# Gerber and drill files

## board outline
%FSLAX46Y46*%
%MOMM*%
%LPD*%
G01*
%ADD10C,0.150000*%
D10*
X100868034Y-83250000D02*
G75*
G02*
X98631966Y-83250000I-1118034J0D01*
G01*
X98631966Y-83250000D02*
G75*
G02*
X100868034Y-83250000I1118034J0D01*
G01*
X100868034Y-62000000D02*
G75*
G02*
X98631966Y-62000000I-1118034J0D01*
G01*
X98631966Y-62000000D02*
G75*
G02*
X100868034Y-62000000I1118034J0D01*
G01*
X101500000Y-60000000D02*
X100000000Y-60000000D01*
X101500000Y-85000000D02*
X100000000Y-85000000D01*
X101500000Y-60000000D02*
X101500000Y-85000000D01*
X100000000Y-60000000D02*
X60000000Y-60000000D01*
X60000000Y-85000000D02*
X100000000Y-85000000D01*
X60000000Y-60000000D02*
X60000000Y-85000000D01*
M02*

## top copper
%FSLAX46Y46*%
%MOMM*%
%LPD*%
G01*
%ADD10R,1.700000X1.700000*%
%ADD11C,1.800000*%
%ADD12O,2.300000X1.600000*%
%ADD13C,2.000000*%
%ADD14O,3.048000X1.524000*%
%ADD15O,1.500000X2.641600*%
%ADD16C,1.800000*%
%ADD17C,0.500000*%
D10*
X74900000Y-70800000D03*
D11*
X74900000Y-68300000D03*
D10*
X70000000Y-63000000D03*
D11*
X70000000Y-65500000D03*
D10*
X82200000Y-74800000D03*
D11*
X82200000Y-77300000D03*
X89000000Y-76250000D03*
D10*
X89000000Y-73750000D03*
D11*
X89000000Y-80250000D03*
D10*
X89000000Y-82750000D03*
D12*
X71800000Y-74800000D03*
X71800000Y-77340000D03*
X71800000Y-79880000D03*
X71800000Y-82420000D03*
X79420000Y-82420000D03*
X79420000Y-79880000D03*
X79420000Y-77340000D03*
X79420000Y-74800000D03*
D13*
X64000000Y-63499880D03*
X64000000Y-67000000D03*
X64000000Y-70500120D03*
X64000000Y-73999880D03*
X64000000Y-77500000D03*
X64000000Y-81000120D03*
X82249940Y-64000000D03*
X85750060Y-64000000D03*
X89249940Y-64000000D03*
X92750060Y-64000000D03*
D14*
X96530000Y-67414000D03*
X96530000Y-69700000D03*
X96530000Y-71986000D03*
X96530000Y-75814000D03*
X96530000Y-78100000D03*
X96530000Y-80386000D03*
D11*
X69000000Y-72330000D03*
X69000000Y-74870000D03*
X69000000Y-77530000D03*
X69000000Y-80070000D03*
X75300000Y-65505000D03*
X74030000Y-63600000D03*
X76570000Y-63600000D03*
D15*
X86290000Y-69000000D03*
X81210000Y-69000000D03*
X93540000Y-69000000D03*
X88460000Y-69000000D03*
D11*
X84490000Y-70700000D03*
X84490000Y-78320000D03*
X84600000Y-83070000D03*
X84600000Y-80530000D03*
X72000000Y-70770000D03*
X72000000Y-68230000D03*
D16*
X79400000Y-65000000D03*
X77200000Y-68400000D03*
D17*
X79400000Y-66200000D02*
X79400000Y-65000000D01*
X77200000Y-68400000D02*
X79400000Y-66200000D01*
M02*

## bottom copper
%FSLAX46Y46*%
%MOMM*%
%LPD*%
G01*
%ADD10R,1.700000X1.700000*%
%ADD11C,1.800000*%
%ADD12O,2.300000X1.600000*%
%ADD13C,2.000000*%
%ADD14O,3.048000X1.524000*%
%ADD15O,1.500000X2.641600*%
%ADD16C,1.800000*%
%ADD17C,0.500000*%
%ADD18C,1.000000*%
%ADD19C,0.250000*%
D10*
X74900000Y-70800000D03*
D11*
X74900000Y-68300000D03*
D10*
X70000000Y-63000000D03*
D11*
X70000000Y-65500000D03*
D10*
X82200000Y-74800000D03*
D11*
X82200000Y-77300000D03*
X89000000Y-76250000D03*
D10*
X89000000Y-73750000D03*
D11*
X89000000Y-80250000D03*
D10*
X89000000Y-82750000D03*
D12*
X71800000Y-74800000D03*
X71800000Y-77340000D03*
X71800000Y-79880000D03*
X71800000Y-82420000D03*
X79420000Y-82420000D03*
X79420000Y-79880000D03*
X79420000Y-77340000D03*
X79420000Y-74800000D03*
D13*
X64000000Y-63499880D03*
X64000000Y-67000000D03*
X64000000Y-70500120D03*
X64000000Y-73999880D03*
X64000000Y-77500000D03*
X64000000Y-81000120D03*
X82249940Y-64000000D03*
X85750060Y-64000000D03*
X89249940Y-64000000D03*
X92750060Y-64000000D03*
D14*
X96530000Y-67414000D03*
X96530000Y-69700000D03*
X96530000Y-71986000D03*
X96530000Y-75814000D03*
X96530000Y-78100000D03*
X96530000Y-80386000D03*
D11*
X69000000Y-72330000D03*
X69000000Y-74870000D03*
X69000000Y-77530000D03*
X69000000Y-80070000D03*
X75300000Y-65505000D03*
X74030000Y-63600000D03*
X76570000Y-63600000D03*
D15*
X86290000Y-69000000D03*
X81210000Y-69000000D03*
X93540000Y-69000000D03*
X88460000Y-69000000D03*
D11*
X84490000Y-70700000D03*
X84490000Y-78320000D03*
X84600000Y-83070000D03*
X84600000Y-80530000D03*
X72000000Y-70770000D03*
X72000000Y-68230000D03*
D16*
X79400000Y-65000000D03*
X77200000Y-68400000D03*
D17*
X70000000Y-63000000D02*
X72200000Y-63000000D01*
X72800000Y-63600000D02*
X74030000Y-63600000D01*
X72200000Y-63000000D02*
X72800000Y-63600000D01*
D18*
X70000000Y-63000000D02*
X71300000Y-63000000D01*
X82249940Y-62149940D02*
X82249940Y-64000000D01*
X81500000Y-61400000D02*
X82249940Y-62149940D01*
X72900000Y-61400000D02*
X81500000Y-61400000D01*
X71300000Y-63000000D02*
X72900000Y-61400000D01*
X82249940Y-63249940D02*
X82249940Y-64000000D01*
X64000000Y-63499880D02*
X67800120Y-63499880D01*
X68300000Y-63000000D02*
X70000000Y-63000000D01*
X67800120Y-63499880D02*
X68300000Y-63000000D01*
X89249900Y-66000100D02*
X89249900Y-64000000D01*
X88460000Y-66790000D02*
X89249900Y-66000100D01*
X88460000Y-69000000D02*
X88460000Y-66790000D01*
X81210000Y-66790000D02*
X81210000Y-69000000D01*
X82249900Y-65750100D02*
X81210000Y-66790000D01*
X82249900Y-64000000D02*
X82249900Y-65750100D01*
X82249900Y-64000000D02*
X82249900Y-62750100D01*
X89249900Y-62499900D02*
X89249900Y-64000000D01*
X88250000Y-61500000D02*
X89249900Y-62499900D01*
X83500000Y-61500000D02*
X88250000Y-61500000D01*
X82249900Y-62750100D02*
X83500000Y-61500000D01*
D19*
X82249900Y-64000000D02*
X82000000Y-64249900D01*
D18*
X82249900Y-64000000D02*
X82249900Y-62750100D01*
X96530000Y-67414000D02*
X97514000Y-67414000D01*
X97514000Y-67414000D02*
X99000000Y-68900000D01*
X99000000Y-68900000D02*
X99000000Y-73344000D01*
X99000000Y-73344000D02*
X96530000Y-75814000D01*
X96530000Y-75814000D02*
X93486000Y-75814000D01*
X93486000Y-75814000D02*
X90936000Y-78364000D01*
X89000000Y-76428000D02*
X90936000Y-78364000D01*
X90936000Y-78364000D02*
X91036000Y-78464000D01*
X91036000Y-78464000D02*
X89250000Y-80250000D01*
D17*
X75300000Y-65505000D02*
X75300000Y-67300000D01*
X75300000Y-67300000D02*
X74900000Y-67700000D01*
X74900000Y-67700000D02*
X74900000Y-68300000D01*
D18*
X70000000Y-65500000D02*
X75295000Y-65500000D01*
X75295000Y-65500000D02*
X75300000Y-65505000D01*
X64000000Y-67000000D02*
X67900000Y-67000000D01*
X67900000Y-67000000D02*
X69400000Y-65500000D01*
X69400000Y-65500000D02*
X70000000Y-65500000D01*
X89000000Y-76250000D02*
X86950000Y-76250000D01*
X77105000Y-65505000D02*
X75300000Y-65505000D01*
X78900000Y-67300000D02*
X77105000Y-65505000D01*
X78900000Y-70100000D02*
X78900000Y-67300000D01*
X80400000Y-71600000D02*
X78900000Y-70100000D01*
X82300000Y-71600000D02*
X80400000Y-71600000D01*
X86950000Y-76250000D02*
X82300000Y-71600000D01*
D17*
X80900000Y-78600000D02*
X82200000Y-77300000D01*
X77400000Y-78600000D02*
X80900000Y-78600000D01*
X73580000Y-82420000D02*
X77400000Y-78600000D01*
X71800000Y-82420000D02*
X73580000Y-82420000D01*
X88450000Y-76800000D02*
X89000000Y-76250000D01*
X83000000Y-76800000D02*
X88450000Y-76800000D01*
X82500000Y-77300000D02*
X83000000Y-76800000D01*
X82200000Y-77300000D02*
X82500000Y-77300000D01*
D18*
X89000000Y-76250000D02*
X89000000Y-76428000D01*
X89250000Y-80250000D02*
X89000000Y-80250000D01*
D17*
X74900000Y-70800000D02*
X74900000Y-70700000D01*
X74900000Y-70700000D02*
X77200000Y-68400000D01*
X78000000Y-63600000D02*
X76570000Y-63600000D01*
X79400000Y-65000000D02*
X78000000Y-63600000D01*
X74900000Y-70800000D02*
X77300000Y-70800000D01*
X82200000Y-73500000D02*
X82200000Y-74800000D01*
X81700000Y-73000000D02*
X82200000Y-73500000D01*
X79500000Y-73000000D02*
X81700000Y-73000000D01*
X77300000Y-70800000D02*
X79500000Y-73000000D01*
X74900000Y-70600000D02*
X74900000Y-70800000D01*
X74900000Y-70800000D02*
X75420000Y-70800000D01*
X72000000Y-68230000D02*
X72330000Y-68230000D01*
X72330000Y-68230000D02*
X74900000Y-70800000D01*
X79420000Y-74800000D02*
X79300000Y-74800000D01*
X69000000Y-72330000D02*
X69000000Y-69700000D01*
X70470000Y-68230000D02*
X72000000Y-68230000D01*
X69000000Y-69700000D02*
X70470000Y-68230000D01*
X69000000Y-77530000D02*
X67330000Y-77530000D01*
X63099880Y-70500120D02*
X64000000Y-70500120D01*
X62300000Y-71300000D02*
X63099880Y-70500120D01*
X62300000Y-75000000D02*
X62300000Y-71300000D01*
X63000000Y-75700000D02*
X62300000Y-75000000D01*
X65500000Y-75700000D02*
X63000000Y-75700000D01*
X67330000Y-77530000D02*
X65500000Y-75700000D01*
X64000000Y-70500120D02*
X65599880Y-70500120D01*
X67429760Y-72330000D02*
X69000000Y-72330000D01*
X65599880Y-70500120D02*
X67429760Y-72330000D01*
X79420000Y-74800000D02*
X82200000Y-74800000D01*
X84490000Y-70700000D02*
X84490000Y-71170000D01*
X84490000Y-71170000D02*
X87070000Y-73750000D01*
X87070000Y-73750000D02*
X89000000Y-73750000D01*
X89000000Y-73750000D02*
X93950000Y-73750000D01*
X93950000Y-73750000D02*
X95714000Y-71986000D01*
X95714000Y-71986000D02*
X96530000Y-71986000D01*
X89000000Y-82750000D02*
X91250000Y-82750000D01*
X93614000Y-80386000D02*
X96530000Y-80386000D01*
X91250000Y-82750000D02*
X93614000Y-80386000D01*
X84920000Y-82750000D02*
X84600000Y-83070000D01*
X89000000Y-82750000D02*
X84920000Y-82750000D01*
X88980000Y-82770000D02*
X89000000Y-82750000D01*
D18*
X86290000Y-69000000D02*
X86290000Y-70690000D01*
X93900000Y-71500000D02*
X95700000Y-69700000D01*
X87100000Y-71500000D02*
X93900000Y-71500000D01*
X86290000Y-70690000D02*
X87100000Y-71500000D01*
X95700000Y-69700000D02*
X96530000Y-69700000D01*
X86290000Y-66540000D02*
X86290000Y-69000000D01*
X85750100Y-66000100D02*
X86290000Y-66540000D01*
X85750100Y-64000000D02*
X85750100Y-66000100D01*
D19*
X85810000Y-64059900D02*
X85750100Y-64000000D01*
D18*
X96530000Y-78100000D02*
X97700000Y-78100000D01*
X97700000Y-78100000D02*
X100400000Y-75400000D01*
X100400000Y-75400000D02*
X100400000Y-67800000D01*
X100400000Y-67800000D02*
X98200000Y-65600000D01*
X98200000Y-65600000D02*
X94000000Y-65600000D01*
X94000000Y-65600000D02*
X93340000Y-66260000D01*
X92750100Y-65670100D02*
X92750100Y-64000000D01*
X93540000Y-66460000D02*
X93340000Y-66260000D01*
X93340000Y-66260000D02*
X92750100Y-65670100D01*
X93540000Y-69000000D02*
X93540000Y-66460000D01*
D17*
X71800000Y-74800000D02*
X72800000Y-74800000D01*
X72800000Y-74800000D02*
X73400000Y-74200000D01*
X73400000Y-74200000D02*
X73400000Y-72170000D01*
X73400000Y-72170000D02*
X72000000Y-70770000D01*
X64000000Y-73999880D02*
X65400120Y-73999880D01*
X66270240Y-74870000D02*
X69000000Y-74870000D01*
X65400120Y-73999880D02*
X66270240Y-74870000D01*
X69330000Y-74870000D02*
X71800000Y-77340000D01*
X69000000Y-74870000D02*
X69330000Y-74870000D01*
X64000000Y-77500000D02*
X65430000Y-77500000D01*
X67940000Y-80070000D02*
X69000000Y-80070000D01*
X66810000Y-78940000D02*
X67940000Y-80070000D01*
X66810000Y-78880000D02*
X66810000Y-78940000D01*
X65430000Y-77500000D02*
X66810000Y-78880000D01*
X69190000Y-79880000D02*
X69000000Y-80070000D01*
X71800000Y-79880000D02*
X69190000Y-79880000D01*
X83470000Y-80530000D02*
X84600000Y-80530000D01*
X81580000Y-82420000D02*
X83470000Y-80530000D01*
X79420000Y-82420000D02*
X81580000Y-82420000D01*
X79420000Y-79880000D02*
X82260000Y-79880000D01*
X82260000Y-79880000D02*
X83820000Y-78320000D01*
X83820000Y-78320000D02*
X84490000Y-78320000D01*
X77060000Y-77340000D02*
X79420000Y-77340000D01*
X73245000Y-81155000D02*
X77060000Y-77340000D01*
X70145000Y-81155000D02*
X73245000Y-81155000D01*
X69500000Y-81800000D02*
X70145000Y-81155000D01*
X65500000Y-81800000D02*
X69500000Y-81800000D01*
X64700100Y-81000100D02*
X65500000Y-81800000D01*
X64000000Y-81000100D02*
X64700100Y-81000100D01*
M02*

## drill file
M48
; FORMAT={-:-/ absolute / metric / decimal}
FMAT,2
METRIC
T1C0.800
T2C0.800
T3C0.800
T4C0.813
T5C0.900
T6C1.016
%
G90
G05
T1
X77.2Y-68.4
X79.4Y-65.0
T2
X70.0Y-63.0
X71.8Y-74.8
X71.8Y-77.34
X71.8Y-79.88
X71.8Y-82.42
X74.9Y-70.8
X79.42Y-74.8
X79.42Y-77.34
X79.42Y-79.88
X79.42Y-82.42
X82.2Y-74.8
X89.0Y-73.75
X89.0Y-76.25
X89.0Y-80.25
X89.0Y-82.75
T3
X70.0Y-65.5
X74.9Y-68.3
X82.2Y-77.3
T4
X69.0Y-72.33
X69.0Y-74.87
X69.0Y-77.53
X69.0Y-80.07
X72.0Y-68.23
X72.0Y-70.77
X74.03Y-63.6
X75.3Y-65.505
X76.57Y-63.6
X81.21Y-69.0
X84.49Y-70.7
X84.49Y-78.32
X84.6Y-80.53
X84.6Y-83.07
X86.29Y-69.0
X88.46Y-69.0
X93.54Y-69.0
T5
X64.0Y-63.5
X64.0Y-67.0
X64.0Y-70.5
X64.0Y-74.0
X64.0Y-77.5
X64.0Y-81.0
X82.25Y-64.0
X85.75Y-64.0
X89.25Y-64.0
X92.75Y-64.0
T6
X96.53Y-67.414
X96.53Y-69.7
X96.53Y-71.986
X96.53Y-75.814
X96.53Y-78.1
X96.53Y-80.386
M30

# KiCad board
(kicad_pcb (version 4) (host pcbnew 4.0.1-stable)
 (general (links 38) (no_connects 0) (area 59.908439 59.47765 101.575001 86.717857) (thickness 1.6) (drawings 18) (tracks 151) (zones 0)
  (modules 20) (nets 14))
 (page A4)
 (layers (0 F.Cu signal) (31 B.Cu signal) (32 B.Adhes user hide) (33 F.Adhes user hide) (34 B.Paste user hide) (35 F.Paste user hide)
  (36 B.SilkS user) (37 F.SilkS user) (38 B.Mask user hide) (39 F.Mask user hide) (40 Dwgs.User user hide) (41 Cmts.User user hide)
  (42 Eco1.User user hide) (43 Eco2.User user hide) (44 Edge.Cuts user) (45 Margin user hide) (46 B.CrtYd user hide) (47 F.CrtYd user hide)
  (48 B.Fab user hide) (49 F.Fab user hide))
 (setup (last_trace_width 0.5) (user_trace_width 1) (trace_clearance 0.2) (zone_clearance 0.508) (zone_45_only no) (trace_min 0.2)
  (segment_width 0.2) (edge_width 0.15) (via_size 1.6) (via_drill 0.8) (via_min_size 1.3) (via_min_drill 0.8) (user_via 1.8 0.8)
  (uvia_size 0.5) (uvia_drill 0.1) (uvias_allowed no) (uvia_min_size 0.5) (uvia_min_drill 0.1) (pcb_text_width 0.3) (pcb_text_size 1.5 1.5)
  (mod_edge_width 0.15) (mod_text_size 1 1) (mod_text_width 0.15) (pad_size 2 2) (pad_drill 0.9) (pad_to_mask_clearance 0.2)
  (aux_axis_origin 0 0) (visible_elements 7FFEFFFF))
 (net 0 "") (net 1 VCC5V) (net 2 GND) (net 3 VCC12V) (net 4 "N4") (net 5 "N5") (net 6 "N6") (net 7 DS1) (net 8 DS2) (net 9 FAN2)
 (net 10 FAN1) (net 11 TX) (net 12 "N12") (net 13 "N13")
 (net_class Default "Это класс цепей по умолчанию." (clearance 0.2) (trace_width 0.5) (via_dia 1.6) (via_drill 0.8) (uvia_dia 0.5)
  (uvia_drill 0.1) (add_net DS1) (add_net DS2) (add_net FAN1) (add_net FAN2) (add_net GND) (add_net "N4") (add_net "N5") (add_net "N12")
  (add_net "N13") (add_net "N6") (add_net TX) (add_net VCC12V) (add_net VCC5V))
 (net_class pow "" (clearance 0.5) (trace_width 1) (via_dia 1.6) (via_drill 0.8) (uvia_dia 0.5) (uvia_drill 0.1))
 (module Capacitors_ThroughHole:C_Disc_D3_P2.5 (layer F.Cu) (at 74.9 70.8 90)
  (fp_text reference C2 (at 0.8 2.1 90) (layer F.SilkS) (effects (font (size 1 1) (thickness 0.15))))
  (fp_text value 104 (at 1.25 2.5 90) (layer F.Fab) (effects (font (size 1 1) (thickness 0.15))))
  (pad 1 thru_hole rect (at 0 0 90) (size 1.7 1.7) (drill 0.8) (layers *.Cu *.Mask F.SilkS) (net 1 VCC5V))
  (pad 2 thru_hole circle (at 2.5 0 90) (size 1.8 1.8) (drill 0.8001) (layers *.Cu *.Mask F.SilkS) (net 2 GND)))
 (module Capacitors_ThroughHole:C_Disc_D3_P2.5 (layer F.Cu) (at 70 63 270)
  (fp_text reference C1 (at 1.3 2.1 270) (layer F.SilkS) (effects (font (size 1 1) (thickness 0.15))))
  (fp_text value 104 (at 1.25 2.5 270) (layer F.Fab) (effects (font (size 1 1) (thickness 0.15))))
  (pad 1 thru_hole rect (at 0 0 270) (size 1.7 1.7) (drill 0.8) (layers *.Cu *.Mask F.SilkS) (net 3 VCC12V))
  (pad 2 thru_hole circle (at 2.5 0 270) (size 1.8 1.8) (drill 0.8001) (layers *.Cu *.Mask F.SilkS) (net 2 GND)))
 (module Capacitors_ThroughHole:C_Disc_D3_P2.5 (layer F.Cu) (at 82.2 74.8 270)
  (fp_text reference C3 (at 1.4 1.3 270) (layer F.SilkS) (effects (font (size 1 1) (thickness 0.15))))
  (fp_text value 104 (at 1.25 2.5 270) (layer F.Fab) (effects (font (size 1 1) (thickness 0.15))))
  (pad 1 thru_hole rect (at 0 0 270) (size 1.7 1.7) (drill 0.8) (layers *.Cu *.Mask F.SilkS) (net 1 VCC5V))
  (pad 2 thru_hole circle (at 2.5 0 270) (size 1.8 1.8) (drill 0.8001) (layers *.Cu *.Mask F.SilkS) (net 2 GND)))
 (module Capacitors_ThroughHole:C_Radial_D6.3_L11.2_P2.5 (layer F.Cu) (at 89 73.75 270)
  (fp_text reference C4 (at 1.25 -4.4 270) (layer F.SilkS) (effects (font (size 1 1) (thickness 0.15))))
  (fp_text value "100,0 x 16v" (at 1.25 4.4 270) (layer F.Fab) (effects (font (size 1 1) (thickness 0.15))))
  (pad 2 thru_hole circle (at 2.5 0 270) (size 1.8 1.8) (drill 0.8) (layers *.Cu *.Mask F.SilkS) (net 2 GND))
  (pad 1 thru_hole rect (at 0 0 270) (size 1.7 1.7) (drill 0.8) (layers *.Cu *.Mask F.SilkS) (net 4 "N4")))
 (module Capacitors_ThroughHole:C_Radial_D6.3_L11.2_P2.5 (layer F.Cu) (at 89 82.75 90)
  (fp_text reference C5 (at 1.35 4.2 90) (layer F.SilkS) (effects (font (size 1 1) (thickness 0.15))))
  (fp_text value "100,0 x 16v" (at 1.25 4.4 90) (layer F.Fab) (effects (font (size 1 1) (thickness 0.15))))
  (pad 2 thru_hole circle (at 2.5 0 90) (size 1.8 1.8) (drill 0.8) (layers *.Cu *.Mask F.SilkS) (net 2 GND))
  (pad 1 thru_hole rect (at 0 0 90) (size 1.7 1.7) (drill 0.8) (layers *.Cu *.Mask F.SilkS) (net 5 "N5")))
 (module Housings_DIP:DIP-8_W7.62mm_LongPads (layer F.Cu) (at 71.8 74.8)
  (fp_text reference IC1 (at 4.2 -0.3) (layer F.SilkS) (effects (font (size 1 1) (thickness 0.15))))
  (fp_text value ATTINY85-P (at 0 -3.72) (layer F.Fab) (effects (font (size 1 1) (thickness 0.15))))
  (pad 1 thru_hole oval (at 0 0) (size 2.3 1.6) (drill 0.8) (layers *.Cu *.Mask F.SilkS) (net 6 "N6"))
  (pad 2 thru_hole oval (at 0 2.54) (size 2.3 1.6) (drill 0.8) (layers *.Cu *.Mask F.SilkS) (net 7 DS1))
  (pad 3 thru_hole oval (at 0 5.08) (size 2.3 1.6) (drill 0.8) (layers *.Cu *.Mask F.SilkS) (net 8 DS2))
  (pad 4 thru_hole oval (at 0 7.62) (size 2.3 1.6) (drill 0.8) (layers *.Cu *.Mask F.SilkS) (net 2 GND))
  (pad 5 thru_hole oval (at 7.62 7.62) (size 2.3 1.6) (drill 0.8) (layers *.Cu *.Mask F.SilkS) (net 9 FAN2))
  (pad 6 thru_hole oval (at 7.62 5.08) (size 2.3 1.6) (drill 0.8) (layers *.Cu *.Mask F.SilkS) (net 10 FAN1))
  (pad 7 thru_hole oval (at 7.62 2.54) (size 2.3 1.6) (drill 0.8) (layers *.Cu *.Mask F.SilkS) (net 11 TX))
  (pad 8 thru_hole oval (at 7.62 0) (size 2.3 1.6) (drill 0.8) (layers *.Cu *.Mask F.SilkS) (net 1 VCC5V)))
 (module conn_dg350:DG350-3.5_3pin (layer F.Cu) (at 64 67 270)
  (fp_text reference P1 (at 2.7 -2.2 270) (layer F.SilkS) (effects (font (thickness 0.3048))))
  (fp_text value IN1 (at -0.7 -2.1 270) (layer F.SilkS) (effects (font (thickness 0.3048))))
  (pad 1 thru_hole circle (at -3.50012 0 270) (size 2 2) (drill 0.9) (layers *.Cu *.Mask F.SilkS) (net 3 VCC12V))
  (pad 2 thru_hole circle (at 0 0 270) (size 2 2) (drill 0.9) (layers *.Cu *.Mask F.SilkS) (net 2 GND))
  (pad 3 thru_hole circle (at 3.50012 0 270) (size 2 2) (drill 0.9) (layers *.Cu *.Mask F.SilkS) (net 1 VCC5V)))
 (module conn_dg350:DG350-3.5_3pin (layer F.Cu) (at 64 77.5 270)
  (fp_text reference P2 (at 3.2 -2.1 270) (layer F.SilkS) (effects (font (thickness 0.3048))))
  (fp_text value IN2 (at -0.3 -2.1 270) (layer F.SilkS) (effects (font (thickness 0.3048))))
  (pad 1 thru_hole circle (at -3.50012 0 270) (size 2 2) (drill 0.9) (layers *.Cu *.Mask F.SilkS) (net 7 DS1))
  (pad 2 thru_hole circle (at 0 0 270) (size 2 2) (drill 0.9) (layers *.Cu *.Mask F.SilkS) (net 8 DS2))
  (pad 3 thru_hole circle (at 3.50012 0 270) (size 2 2) (drill 0.9) (layers *.Cu *.Mask F.SilkS) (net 11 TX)))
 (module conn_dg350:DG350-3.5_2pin (layer F.Cu) (at 84 64)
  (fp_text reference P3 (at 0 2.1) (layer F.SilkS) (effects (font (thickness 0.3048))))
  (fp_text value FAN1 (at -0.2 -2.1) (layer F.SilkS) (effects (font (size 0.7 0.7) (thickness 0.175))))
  (pad 1 thru_hole circle (at -1.75006 0) (size 2 2) (drill 0.9) (layers *.Cu *.Mask F.SilkS) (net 3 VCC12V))
  (pad 2 thru_hole circle (at 1.75006 0) (size 2 2) (drill 0.9) (layers *.Cu *.Mask F.SilkS) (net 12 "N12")))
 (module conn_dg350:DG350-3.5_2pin (layer F.Cu) (at 91 64)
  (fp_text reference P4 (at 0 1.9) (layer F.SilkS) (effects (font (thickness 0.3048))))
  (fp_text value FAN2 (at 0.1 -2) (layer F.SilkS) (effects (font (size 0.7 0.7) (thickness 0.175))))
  (pad 1 thru_hole circle (at -1.75006 0) (size 2 2) (drill 0.9) (layers *.Cu *.Mask F.SilkS) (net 3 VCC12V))
  (pad 2 thru_hole circle (at 1.75006 0) (size 2 2) (drill 0.9) (layers *.Cu *.Mask F.SilkS) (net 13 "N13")))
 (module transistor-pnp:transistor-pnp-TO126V (layer F.Cu) (at 97.8 69.7 270)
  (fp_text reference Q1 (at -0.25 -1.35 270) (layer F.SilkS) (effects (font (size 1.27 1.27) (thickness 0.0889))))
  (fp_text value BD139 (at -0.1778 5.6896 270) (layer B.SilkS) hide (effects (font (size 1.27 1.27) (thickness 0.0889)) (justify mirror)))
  (pad 1 thru_hole oval (at -2.286 1.27 270) (size 1.524 3.048) (drill 1.016) (layers *.Cu F.Paste F.SilkS F.Mask) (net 2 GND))
  (pad 2 thru_hole oval (at 0 1.27 270) (size 1.524 3.048) (drill 1.016) (layers *.Cu F.Paste F.SilkS F.Mask) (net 12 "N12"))
  (pad 3 thru_hole oval (at 2.286 1.27 270) (size 1.524 3.048) (drill 1.016) (layers *.Cu F.Paste F.SilkS F.Mask) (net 4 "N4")))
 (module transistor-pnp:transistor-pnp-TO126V (layer F.Cu) (at 97.8 78.1 270)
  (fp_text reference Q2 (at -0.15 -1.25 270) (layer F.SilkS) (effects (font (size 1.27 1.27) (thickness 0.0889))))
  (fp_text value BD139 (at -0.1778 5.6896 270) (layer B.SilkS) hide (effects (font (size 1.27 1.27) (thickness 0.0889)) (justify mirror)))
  (pad 1 thru_hole oval (at -2.286 1.27 270) (size 1.524 3.048) (drill 1.016) (layers *.Cu F.Paste F.SilkS F.Mask) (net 2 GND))
  (pad 2 thru_hole oval (at 0 1.27 270) (size 1.524 3.048) (drill 1.016) (layers *.Cu F.Paste F.SilkS F.Mask) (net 13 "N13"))
  (pad 3 thru_hole oval (at 2.286 1.27 270) (size 1.524 3.048) (drill 1.016) (layers *.Cu F.Paste F.SilkS F.Mask) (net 5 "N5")))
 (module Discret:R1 (layer F.Cu) (at 69 73.6 270)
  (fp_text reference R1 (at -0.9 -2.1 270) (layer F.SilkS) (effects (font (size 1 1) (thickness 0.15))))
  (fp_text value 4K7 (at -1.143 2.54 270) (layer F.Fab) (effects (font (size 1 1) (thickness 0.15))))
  (pad 1 thru_hole circle (at -1.27 0 270) (size 1.8 1.8) (drill 0.8128) (layers *.Cu *.Mask F.SilkS) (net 1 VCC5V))
  (pad 2 thru_hole circle (at 1.27 0 270) (size 1.8 1.8) (drill 0.8128) (layers *.Cu *.Mask F.SilkS) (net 7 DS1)))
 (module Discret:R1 (layer F.Cu) (at 69 78.8 270)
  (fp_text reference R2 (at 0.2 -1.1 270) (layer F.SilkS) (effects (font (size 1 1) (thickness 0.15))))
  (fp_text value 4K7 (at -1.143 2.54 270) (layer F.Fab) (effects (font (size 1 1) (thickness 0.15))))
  (pad 1 thru_hole circle (at -1.27 0 270) (size 1.8 1.8) (drill 0.8128) (layers *.Cu *.Mask F.SilkS) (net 1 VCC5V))
  (pad 2 thru_hole circle (at 1.27 0 270) (size 1.8 1.8) (drill 0.8128) (layers *.Cu *.Mask F.SilkS) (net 8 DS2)))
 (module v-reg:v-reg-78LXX (layer F.Cu) (at 75.3 63.6 180)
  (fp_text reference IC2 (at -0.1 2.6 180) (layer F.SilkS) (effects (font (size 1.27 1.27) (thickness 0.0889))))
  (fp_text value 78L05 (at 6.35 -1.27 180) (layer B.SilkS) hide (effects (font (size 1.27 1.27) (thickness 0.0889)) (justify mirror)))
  (pad GND thru_hole circle (at 0 -1.905 180) (size 1.8 1.8) (drill 0.8128) (layers *.Cu F.Paste F.SilkS F.Mask) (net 2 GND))
  (pad IN thru_hole circle (at 1.27 0 180) (size 1.8 1.8) (drill 0.8128) (layers *.Cu F.Paste F.SilkS F.Mask) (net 3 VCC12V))
  (pad OUT thru_hole circle (at -1.27 0 180) (size 1.8 1.8) (drill 0.8128) (layers *.Cu F.Paste F.SilkS F.Mask) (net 1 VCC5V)))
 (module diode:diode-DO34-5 (layer F.Cu) (at 83.75 69)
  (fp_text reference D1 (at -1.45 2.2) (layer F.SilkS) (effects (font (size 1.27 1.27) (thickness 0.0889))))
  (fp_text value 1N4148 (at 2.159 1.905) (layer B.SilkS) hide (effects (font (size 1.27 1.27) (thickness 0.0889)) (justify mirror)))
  (pad 2 thru_hole oval (at 2.54 0) (size 1.5 2.6416) (drill 0.8128) (layers *.Cu F.Paste F.SilkS F.Mask) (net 12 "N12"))
  (pad 1 thru_hole oval (at -2.54 0) (size 1.5 2.6416) (drill 0.8128) (layers *.Cu F.Paste F.SilkS F.Mask) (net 3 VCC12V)))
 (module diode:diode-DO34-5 (layer F.Cu) (at 91 69)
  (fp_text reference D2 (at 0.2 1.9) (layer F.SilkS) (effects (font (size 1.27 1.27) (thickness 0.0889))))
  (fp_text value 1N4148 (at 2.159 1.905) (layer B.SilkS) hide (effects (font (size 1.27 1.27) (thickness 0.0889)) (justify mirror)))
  (pad 2 thru_hole oval (at 2.54 0) (size 1.5 2.6416) (drill 0.8128) (layers *.Cu F.Paste F.SilkS F.Mask) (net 13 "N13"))
  (pad 1 thru_hole oval (at -2.54 0) (size 1.5 2.6416) (drill 0.8128) (layers *.Cu F.Paste F.SilkS F.Mask) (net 3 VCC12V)))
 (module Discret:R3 (layer F.Cu) (at 84.49 74.51 270)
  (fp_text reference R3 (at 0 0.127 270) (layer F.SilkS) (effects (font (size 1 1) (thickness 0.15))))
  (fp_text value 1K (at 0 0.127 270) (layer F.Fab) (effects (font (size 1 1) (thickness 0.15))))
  (pad 1 thru_hole circle (at -3.81 0 270) (size 1.8 1.8) (drill 0.8128) (layers *.Cu *.Mask F.SilkS) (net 4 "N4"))
  (pad 2 thru_hole circle (at 3.81 0 270) (size 1.8 1.8) (drill 0.8128) (layers *.Cu *.Mask F.SilkS) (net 10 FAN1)))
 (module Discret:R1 (layer F.Cu) (at 84.6 81.8 90)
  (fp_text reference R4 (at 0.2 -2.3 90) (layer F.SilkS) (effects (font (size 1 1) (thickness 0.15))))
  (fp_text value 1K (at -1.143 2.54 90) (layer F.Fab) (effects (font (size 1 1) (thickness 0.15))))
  (pad 1 thru_hole circle (at -1.27 0 90) (size 1.8 1.8) (drill 0.8128) (layers *.Cu *.Mask F.SilkS) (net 5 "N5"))
  (pad 2 thru_hole circle (at 1.27 0 90) (size 1.8 1.8) (drill 0.8128) (layers *.Cu *.Mask F.SilkS) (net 9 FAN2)))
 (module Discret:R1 (layer F.Cu) (at 72 69.5 90)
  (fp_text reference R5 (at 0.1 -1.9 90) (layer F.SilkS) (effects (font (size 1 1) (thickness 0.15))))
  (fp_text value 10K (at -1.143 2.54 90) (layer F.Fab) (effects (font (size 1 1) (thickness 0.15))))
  (pad 1 thru_hole circle (at -1.27 0 90) (size 1.8 1.8) (drill 0.8128) (layers *.Cu *.Mask F.SilkS) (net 6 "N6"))
  (pad 2 thru_hole circle (at 1.27 0 90) (size 1.8 1.8) (drill 0.8128) (layers *.Cu *.Mask F.SilkS) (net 1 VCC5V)))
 (gr_circle (center 99.75 83.25) (end 100.75 82.75) (layer Edge.Cuts) (width 0.15))
 (gr_circle (center 99.75 62) (end 100.75 61.5) (layer Edge.Cuts) (width 0.15))
 (gr_line (start 101.5 60) (end 100 60) (angle 90) (layer Edge.Cuts) (width 0.15))
 (gr_line (start 101.5 85) (end 100 85) (angle 90) (layer Edge.Cuts) (width 0.15))
 (gr_line (start 101.5 60) (end 101.5 85) (angle 90) (layer Edge.Cuts) (width 0.15))
 (gr_line (start 100 60) (end 60 60) (angle 90) (layer Edge.Cuts) (width 0.15))
 (gr_line (start 60 85) (end 100 85) (angle 90) (layer Edge.Cuts) (width 0.15))
 (gr_line (start 60 60) (end 60 85) (angle 90) (layer Edge.Cuts) (width 0.15))
 (segment (start 70 63) (end 72.2 63) (width 0.5) (layer B.Cu) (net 3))
 (segment (start 72.8 63.6) (end 74.03 63.6) (width 0.5) (layer B.Cu) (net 3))
 (segment (start 72.2 63) (end 72.8 63.6) (width 0.5) (layer B.Cu) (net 3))
 (segment (start 70 63) (end 71.3 63) (width 1) (layer B.Cu) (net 3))
 (segment (start 82.24994 62.14994) (end 82.24994 64) (width 1) (layer B.Cu) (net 3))
 (segment (start 81.5 61.4) (end 82.24994 62.14994) (width 1) (layer B.Cu) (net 3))
 (segment (start 72.9 61.4) (end 81.5 61.4) (width 1) (layer B.Cu) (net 3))
 (segment (start 71.3 63) (end 72.9 61.4) (width 1) (layer B.Cu) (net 3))
 (segment (start 82.24994 63.24994) (end 82.24994 64) (width 1) (layer B.Cu) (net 3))
 (segment (start 64 63.49988) (end 67.80012 63.49988) (width 1) (layer B.Cu) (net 3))
 (segment (start 68.3 63) (end 70 63) (width 1) (layer B.Cu) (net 3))
 (segment (start 67.80012 63.49988) (end 68.3 63) (width 1) (layer B.Cu) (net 3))
 (segment (start 89.2499 66.0001) (end 89.2499 64) (width 1) (layer B.Cu) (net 3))
 (segment (start 88.46 66.79) (end 89.2499 66.0001) (width 1) (layer B.Cu) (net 3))
 (segment (start 88.46 69) (end 88.46 66.79) (width 1) (layer B.Cu) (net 3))
 (segment (start 81.21 66.79) (end 81.21 69) (width 1) (layer B.Cu) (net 3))
 (segment (start 82.2499 65.7501) (end 81.21 66.79) (width 1) (layer B.Cu) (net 3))
 (segment (start 82.2499 64) (end 82.2499 65.7501) (width 1) (layer B.Cu) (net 3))
 (segment (start 82.2499 64) (end 82.2499 62.7501) (width 1) (layer B.Cu) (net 3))
 (segment (start 89.2499 62.4999) (end 89.2499 64) (width 1) (layer B.Cu) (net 3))
 (segment (start 88.25 61.5) (end 89.2499 62.4999) (width 1) (layer B.Cu) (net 3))
 (segment (start 83.5 61.5) (end 88.25 61.5) (width 1) (layer B.Cu) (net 3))
 (segment (start 82.2499 62.7501) (end 83.5 61.5) (width 1) (layer B.Cu) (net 3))
 (segment (start 82.2499 64) (end 82 64.2499) (width 0.25) (layer B.Cu) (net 3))
 (segment (start 82.2499 64) (end 82.2499 62.7501) (width 1) (layer B.Cu) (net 3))
 (segment (start 96.53 67.414) (end 97.514 67.414) (width 1) (layer B.Cu) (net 2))
 (segment (start 97.514 67.414) (end 99 68.9) (width 1) (layer B.Cu) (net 2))
 (segment (start 99 68.9) (end 99 73.344) (width 1) (layer B.Cu) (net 2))
 (segment (start 99 73.344) (end 96.53 75.814) (width 1) (layer B.Cu) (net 2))
 (segment (start 96.53 75.814) (end 93.486 75.814) (width 1) (layer B.Cu) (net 2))
 (segment (start 93.486 75.814) (end 90.936 78.364) (width 1) (layer B.Cu) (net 2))
 (segment (start 89 76.428) (end 90.936 78.364) (width 1) (layer B.Cu) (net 2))
 (segment (start 90.936 78.364) (end 91.036 78.464) (width 1) (layer B.Cu) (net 2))
 (segment (start 91.036 78.464) (end 89.25 80.25) (width 1) (layer B.Cu) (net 2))
 (segment (start 75.3 65.505) (end 75.3 67.3) (width 0.5) (layer B.Cu) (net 2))
 (segment (start 75.3 67.3) (end 74.9 67.7) (width 0.5) (layer B.Cu) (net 2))
 (segment (start 74.9 67.7) (end 74.9 68.3) (width 0.5) (layer B.Cu) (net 2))
 (segment (start 70 65.5) (end 75.295 65.5) (width 1) (layer B.Cu) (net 2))
 (segment (start 75.295 65.5) (end 75.3 65.505) (width 1) (layer B.Cu) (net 2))
 (segment (start 64 67) (end 67.9 67) (width 1) (layer B.Cu) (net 2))
 (segment (start 67.9 67) (end 69.4 65.5) (width 1) (layer B.Cu) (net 2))
 (segment (start 69.4 65.5) (end 70 65.5) (width 1) (layer B.Cu) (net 2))
 (segment (start 89 76.25) (end 86.95 76.25) (width 1) (layer B.Cu) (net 2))
 (segment (start 77.105 65.505) (end 75.3 65.505) (width 1) (layer B.Cu) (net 2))
 (segment (start 78.9 67.3) (end 77.105 65.505) (width 1) (layer B.Cu) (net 2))
 (segment (start 78.9 70.1) (end 78.9 67.3) (width 1) (layer B.Cu) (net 2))
 (segment (start 80.4 71.6) (end 78.9 70.1) (width 1) (layer B.Cu) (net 2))
 (segment (start 82.3 71.6) (end 80.4 71.6) (width 1) (layer B.Cu) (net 2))
 (segment (start 86.95 76.25) (end 82.3 71.6) (width 1) (layer B.Cu) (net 2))
 (segment (start 80.9 78.6) (end 82.2 77.3) (width 0.5) (layer B.Cu) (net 2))
 (segment (start 77.4 78.6) (end 80.9 78.6) (width 0.5) (layer B.Cu) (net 2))
 (segment (start 73.58 82.42) (end 77.4 78.6) (width 0.5) (layer B.Cu) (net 2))
 (segment (start 71.8 82.42) (end 73.58 82.42) (width 0.5) (layer B.Cu) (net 2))
 (segment (start 88.45 76.8) (end 89 76.25) (width 0.5) (layer B.Cu) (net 2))
 (segment (start 83 76.8) (end 88.45 76.8) (width 0.5) (layer B.Cu) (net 2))
 (segment (start 82.5 77.3) (end 83 76.8) (width 0.5) (layer B.Cu) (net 2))
 (segment (start 82.2 77.3) (end 82.5 77.3) (width 0.5) (layer B.Cu) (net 2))
 (segment (start 89 76.25) (end 89 76.428) (width 1) (layer B.Cu) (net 2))
 (segment (start 89.25 80.25) (end 89 80.25) (width 1) (layer B.Cu) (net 2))
 (segment (start 74.9 70.8) (end 74.9 70.7) (width 0.5) (layer B.Cu) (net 1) (status C00000))
 (segment (start 74.9 70.7) (end 77.2 68.4) (width 0.5) (layer B.Cu) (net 1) (status 400000))
 (segment (start 78 63.6) (end 76.57 63.6) (width 0.5) (layer B.Cu) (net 1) (status 800000))
 (segment (start 79.4 65) (end 78 63.6) (width 0.5) (layer B.Cu) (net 1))
 (via (at 79.4 65) (size 1.8) (drill 0.8) (layers F.Cu B.Cu) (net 1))
 (segment (start 79.4 66.2) (end 79.4 65) (width 0.5) (layer F.Cu) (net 1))
 (segment (start 77.2 68.4) (end 79.4 66.2) (width 0.5) (layer F.Cu) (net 1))
 (via (at 77.2 68.4) (size 1.8) (drill 0.8) (layers F.Cu B.Cu) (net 1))
 (segment (start 74.9 70.8) (end 77.3 70.8) (width 0.5) (layer B.Cu) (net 1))
 (segment (start 82.2 73.5) (end 82.2 74.8) (width 0.5) (layer B.Cu) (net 1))
 (segment (start 81.7 73) (end 82.2 73.5) (width 0.5) (layer B.Cu) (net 1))
 (segment (start 79.5 73) (end 81.7 73) (width 0.5) (layer B.Cu) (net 1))
 (segment (start 77.3 70.8) (end 79.5 73) (width 0.5) (layer B.Cu) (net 1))
 (segment (start 74.9 70.6) (end 74.9 70.8) (width 0.5) (layer B.Cu) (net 1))
 (segment (start 74.9 70.8) (end 75.42 70.8) (width 0.5) (layer B.Cu) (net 1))
 (segment (start 72 68.23) (end 72.33 68.23) (width 0.5) (layer B.Cu) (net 1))
 (segment (start 72.33 68.23) (end 74.9 70.8) (width 0.5) (layer B.Cu) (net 1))
 (segment (start 79.42 74.8) (end 79.3 74.8) (width 0.5) (layer B.Cu) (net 1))
 (segment (start 69 72.33) (end 69 69.7) (width 0.5) (layer B.Cu) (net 1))
 (segment (start 70.47 68.23) (end 72 68.23) (width 0.5) (layer B.Cu) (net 1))
 (segment (start 69 69.7) (end 70.47 68.23) (width 0.5) (layer B.Cu) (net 1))
 (segment (start 69 77.53) (end 67.33 77.53) (width 0.5) (layer B.Cu) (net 1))
 (segment (start 63.09988 70.50012) (end 64 70.50012) (width 0.5) (layer B.Cu) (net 1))
 (segment (start 62.3 71.3) (end 63.09988 70.50012) (width 0.5) (layer B.Cu) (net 1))
 (segment (start 62.3 75) (end 62.3 71.3) (width 0.5) (layer B.Cu) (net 1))
 (segment (start 63 75.7) (end 62.3 75) (width 0.5) (layer B.Cu) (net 1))
 (segment (start 65.5 75.7) (end 63 75.7) (width 0.5) (layer B.Cu) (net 1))
 (segment (start 67.33 77.53) (end 65.5 75.7) (width 0.5) (layer B.Cu) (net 1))
 (segment (start 64 70.50012) (end 65.59988 70.50012) (width 0.5) (layer B.Cu) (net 1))
 (segment (start 67.42976 72.33) (end 69 72.33) (width 0.5) (layer B.Cu) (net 1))
 (segment (start 65.59988 70.50012) (end 67.42976 72.33) (width 0.5) (layer B.Cu) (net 1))
 (segment (start 79.42 74.8) (end 82.2 74.8) (width 0.5) (layer B.Cu) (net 1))
 (segment (start 84.49 70.7) (end 84.49 71.17) (width 0.5) (layer B.Cu) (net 4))
 (segment (start 84.49 71.17) (end 87.07 73.75) (width 0.5) (layer B.Cu) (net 4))
 (segment (start 87.07 73.75) (end 89 73.75) (width 0.5) (layer B.Cu) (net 4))
 (segment (start 89 73.75) (end 93.95 73.75) (width 0.5) (layer B.Cu) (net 4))
 (segment (start 93.95 73.75) (end 95.714 71.986) (width 0.5) (layer B.Cu) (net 4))
 (segment (start 95.714 71.986) (end 96.53 71.986) (width 0.5) (layer B.Cu) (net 4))
 (segment (start 89 82.75) (end 91.25 82.75) (width 0.5) (layer B.Cu) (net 5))
 (segment (start 93.614 80.386) (end 96.53 80.386) (width 0.5) (layer B.Cu) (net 5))
 (segment (start 91.25 82.75) (end 93.614 80.386) (width 0.5) (layer B.Cu) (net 5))
 (segment (start 84.92 82.75) (end 84.6 83.07) (width 0.5) (layer B.Cu) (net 5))
 (segment (start 89 82.75) (end 84.92 82.75) (width 0.5) (layer B.Cu) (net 5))
 (segment (start 88.98 82.77) (end 89 82.75) (width 0.5) (layer B.Cu) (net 5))
 (segment (start 86.29 69) (end 86.29 70.69) (width 1) (layer B.Cu) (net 12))
 (segment (start 93.9 71.5) (end 95.7 69.7) (width 1) (layer B.Cu) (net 12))
 (segment (start 87.1 71.5) (end 93.9 71.5) (width 1) (layer B.Cu) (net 12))
 (segment (start 86.29 70.69) (end 87.1 71.5) (width 1) (layer B.Cu) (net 12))
 (segment (start 95.7 69.7) (end 96.53 69.7) (width 1) (layer B.Cu) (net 12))
 (segment (start 86.29 66.54) (end 86.29 69) (width 1) (layer B.Cu) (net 12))
 (segment (start 85.7501 66.0001) (end 86.29 66.54) (width 1) (layer B.Cu) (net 12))
 (segment (start 85.7501 64) (end 85.7501 66.0001) (width 1) (layer B.Cu) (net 12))
 (segment (start 85.81 64.0599) (end 85.7501 64) (width 0.25) (layer B.Cu) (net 12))
 (segment (start 96.53 78.1) (end 97.7 78.1) (width 1) (layer B.Cu) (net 13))
 (segment (start 97.7 78.1) (end 100.4 75.4) (width 1) (layer B.Cu) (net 13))
 (segment (start 100.4 75.4) (end 100.4 67.8) (width 1) (layer B.Cu) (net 13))
 (segment (start 100.4 67.8) (end 98.2 65.6) (width 1) (layer B.Cu) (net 13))
 (segment (start 98.2 65.6) (end 94 65.6) (width 1) (layer B.Cu) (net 13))
 (segment (start 94 65.6) (end 93.34 66.26) (width 1) (layer B.Cu) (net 13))
 (segment (start 92.7501 65.6701) (end 92.7501 64) (width 1) (layer B.Cu) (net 13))
 (segment (start 93.54 66.46) (end 93.34 66.26) (width 1) (layer B.Cu) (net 13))
 (segment (start 93.34 66.26) (end 92.7501 65.6701) (width 1) (layer B.Cu) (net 13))
 (segment (start 93.54 69) (end 93.54 66.46) (width 1) (layer B.Cu) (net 13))
 (segment (start 71.8 74.8) (end 72.8 74.8) (width 0.5) (layer B.Cu) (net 6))
 (segment (start 72.8 74.8) (end 73.4 74.2) (width 0.5) (layer B.Cu) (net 6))
 (segment (start 73.4 74.2) (end 73.4 72.17) (width 0.5) (layer B.Cu) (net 6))
 (segment (start 73.4 72.17) (end 72 70.77) (width 0.5) (layer B.Cu) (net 6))
 (segment (start 64 73.99988) (end 65.40012 73.99988) (width 0.5) (layer B.Cu) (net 7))
 (segment (start 66.27024 74.87) (end 69 74.87) (width 0.5) (layer B.Cu) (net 7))
 (segment (start 65.40012 73.99988) (end 66.27024 74.87) (width 0.5) (layer B.Cu) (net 7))
 (segment (start 69.33 74.87) (end 71.8 77.34) (width 0.5) (layer B.Cu) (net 7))
 (segment (start 69 74.87) (end 69.33 74.87) (width 0.5) (layer B.Cu) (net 7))
 (segment (start 64 77.5) (end 65.43 77.5) (width 0.5) (layer B.Cu) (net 8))
 (segment (start 67.94 80.07) (end 69 80.07) (width 0.5) (layer B.Cu) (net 8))
 (segment (start 66.81 78.94) (end 67.94 80.07) (width 0.5) (layer B.Cu) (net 8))
 (segment (start 66.81 78.88) (end 66.81 78.94) (width 0.5) (layer B.Cu) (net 8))
 (segment (start 65.43 77.5) (end 66.81 78.88) (width 0.5) (layer B.Cu) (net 8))
 (segment (start 69.19 79.88) (end 69 80.07) (width 0.5) (layer B.Cu) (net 8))
 (segment (start 71.8 79.88) (end 69.19 79.88) (width 0.5) (layer B.Cu) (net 8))
 (segment (start 83.47 80.53) (end 84.6 80.53) (width 0.5) (layer B.Cu) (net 9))
 (segment (start 81.58 82.42) (end 83.47 80.53) (width 0.5) (layer B.Cu) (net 9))
 (segment (start 79.42 82.42) (end 81.58 82.42) (width 0.5) (layer B.Cu) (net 9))
 (segment (start 79.42 79.88) (end 82.26 79.88) (width 0.5) (layer B.Cu) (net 10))
 (segment (start 82.26 79.88) (end 83.82 78.32) (width 0.5) (layer B.Cu) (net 10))
 (segment (start 83.82 78.32) (end 84.49 78.32) (width 0.5) (layer B.Cu) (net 10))
 (segment (start 77.06 77.34) (end 79.42 77.34) (width 0.5) (layer B.Cu) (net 11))
 (segment (start 73.245 81.155) (end 77.06 77.34) (width 0.5) (layer B.Cu) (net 11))
 (segment (start 70.145 81.155) (end 73.245 81.155) (width 0.5) (layer B.Cu) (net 11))
 (segment (start 69.5 81.8) (end 70.145 81.155) (width 0.5) (layer B.Cu) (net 11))
 (segment (start 65.5 81.8) (end 69.5 81.8) (width 0.5) (layer B.Cu) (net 11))
 (segment (start 64.7001 81.0001) (end 65.5 81.8) (width 0.5) (layer B.Cu) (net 11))
 (segment (start 64 81.0001) (end 64.7001 81.0001) (width 0.5) (layer B.Cu) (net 11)))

